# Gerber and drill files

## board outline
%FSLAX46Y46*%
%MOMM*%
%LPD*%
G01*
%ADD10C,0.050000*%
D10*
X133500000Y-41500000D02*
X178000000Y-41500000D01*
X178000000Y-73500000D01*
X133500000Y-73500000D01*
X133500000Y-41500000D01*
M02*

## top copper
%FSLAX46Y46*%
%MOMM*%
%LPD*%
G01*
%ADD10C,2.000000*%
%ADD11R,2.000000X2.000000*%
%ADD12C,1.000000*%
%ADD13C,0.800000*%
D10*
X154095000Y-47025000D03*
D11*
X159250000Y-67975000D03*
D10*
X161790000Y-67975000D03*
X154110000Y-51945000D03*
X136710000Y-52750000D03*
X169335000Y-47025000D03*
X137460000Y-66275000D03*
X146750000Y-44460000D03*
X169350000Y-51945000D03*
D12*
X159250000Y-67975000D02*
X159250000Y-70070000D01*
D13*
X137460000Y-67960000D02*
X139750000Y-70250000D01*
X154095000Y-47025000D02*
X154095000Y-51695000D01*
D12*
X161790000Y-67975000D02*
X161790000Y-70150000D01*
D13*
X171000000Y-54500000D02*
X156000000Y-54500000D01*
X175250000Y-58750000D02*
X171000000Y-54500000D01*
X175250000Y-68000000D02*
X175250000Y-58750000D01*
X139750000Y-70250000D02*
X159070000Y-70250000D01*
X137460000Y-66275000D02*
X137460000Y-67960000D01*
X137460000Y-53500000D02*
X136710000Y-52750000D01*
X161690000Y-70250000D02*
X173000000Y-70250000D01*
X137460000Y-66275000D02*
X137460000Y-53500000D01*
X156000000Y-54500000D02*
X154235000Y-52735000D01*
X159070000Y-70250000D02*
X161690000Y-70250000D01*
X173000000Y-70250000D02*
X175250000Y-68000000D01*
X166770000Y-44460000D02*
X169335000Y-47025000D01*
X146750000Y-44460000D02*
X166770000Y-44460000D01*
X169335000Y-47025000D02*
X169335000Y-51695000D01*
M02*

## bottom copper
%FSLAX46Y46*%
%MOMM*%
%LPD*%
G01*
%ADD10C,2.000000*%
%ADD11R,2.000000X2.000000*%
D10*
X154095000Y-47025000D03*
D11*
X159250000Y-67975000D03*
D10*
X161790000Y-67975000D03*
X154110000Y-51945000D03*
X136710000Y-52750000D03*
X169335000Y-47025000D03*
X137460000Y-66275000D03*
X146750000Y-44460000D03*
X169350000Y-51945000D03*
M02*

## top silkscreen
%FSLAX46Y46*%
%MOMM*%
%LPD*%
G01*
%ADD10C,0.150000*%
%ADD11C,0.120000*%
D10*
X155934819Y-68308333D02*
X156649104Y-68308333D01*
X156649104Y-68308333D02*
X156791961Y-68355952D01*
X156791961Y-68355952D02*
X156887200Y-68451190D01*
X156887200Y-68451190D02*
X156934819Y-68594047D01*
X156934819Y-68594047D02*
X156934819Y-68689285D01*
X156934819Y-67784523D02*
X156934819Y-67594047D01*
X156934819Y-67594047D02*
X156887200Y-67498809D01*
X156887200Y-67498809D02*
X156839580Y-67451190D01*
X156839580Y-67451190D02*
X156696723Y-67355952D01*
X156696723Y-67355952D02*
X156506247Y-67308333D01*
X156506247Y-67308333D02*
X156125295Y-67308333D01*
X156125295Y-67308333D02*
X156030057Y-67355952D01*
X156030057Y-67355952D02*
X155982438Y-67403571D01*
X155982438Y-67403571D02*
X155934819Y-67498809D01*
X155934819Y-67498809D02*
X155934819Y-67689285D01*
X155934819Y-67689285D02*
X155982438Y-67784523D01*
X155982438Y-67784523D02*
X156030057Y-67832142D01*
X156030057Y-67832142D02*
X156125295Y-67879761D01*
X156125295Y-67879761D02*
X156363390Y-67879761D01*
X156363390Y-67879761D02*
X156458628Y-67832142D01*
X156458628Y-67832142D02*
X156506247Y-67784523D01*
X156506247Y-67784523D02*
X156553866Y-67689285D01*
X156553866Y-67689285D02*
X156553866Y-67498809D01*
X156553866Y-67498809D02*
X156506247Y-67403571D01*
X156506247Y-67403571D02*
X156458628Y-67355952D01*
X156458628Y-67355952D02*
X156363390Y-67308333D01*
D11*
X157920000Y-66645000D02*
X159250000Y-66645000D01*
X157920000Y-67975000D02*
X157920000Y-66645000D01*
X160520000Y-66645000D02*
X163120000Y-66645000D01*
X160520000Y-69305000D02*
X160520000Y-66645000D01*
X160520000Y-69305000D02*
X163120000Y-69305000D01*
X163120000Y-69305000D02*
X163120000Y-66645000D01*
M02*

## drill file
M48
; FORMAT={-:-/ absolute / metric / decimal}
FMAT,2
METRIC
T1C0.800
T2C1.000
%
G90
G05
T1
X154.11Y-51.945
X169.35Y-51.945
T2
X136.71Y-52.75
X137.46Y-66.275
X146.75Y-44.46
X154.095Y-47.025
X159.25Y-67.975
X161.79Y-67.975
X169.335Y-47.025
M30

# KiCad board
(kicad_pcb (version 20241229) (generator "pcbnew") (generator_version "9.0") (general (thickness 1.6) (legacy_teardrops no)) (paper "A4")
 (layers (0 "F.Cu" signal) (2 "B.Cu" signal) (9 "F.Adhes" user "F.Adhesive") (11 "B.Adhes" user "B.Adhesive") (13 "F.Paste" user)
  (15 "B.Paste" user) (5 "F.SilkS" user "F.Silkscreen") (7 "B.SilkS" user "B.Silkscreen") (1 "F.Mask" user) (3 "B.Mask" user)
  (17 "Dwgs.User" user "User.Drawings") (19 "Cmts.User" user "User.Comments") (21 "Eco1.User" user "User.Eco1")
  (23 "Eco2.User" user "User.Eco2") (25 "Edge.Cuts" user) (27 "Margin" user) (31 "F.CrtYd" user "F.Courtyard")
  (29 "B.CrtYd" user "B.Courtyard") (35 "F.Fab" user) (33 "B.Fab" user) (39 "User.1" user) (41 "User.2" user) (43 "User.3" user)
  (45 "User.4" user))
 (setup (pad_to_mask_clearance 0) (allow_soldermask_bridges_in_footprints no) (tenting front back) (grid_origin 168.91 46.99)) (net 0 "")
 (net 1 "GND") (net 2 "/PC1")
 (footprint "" (layer "F.Cu") (at 149.16 46.74)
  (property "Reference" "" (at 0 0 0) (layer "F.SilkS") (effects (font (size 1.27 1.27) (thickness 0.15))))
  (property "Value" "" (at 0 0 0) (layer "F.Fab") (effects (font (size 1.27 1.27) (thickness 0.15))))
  (pad "8" thru_hole circle (at 4.935 0.285 270) (size 2 2) (drill 1) (layers "*.Cu" "*.Mask") (remove_unused_layers no) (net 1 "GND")))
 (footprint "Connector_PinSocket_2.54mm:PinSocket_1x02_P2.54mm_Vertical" (layer "F.Cu") (at 159.25 67.975 90)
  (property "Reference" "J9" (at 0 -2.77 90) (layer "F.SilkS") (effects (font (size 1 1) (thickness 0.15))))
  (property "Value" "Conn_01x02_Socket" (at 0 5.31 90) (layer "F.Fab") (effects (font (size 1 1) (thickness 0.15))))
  (fp_line (start 1.33 -1.33) (end 1.33 0) (stroke (width 0.12) (type solid)) (layer "F.SilkS"))
  (fp_line (start 0 -1.33) (end 1.33 -1.33) (stroke (width 0.12) (type solid)) (layer "F.SilkS"))
  (fp_line (start 1.33 1.27) (end 1.33 3.87) (stroke (width 0.12) (type solid)) (layer "F.SilkS"))
  (fp_line (start -1.33 1.27) (end 1.33 1.27) (stroke (width 0.12) (type solid)) (layer "F.SilkS"))
  (fp_line (start -1.33 1.27) (end -1.33 3.87) (stroke (width 0.12) (type solid)) (layer "F.SilkS"))
  (fp_line (start -1.33 3.87) (end 1.33 3.87) (stroke (width 0.12) (type solid)) (layer "F.SilkS"))
  (pad "1" thru_hole rect (at 0 0 90) (size 2 2) (drill 1) (layers "*.Cu" "*.Mask") (remove_unused_layers no) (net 1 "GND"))
  (pad "2" thru_hole circle (at 0 2.54 90) (size 2 2) (drill 1) (layers "*.Cu" "*.Mask") (remove_unused_layers no) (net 1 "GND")))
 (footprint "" (layer "F.Cu") (at 150.41 50.24)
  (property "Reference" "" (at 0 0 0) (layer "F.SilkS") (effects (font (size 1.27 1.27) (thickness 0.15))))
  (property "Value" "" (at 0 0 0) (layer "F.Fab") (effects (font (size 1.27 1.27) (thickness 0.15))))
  (pad "8" thru_hole circle (at 3.7 1.705 270) (size 2 2) (drill 0.8) (layers "*.Cu" "*.Mask") (remove_unused_layers no) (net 1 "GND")))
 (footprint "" (layer "F.Cu") (at 130.16 50.24)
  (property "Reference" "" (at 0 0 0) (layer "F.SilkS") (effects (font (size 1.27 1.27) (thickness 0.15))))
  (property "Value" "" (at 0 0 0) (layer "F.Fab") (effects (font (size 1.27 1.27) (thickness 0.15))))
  (pad "2" thru_hole circle (at 6.55 2.51 270) (size 2 2) (drill 1) (layers "*.Cu" "*.Mask") (remove_unused_layers no) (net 1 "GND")))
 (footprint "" (layer "F.Cu") (at 169.335 43.24)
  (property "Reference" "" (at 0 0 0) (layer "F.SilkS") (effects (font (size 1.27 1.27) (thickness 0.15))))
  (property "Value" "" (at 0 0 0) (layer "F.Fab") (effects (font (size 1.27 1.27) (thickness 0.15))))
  (pad "2" thru_hole circle (at 0 3.785 270) (size 2 2) (drill 1) (layers "*.Cu" "*.Mask") (remove_unused_layers no) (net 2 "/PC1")))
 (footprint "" (layer "F.Cu") (at 134.91 61.99)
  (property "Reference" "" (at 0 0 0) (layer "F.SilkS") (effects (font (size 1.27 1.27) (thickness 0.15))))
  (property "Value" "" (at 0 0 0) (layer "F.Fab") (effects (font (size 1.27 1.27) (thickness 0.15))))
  (pad "2" thru_hole circle (at 2.55 4.285 270) (size 2 2) (drill 1) (layers "*.Cu" "*.Mask") (remove_unused_layers no) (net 1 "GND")))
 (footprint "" (layer "F.Cu") (at 142.66 44.46)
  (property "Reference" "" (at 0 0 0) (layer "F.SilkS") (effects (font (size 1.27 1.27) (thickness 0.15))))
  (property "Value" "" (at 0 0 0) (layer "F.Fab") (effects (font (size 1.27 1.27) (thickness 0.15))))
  (pad "2" thru_hole circle (at 4.09 0 180) (size 2 2) (drill 1) (layers "*.Cu" "*.Mask") (remove_unused_layers no) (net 2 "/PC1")))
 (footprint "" (layer "F.Cu") (at 175.41 49.24)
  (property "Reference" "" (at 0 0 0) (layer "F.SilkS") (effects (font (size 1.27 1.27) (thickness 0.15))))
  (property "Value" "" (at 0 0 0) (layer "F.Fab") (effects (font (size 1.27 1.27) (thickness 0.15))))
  (pad "2" thru_hole circle (at -6.06 2.705 270) (size 2 2) (drill 0.8) (layers "*.Cu" "*.Mask") (remove_unused_layers no) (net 2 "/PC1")))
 (gr_rect (start 133.5 41.5) (end 178 73.5) (stroke (width 0.05) (type default)) (fill no) (locked yes) (layer "Edge.Cuts"))
 (segment (start 159.25 67.975) (end 159.25 70.07) (width 1) (locked yes) (layer "F.Cu") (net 1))
 (segment (start 137.46 67.96) (end 139.75 70.25) (width 0.8) (locked yes) (layer "F.Cu") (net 1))
 (segment (start 154.095 47.025) (end 154.095 51.695) (width 0.8) (locked yes) (layer "F.Cu") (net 1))
 (segment (start 161.79 67.975) (end 161.79 70.15) (width 1) (locked yes) (layer "F.Cu") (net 1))
 (segment (start 171 54.5) (end 156 54.5) (width 0.8) (locked yes) (layer "F.Cu") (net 1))
 (segment (start 175.25 58.75) (end 171 54.5) (width 0.8) (locked yes) (layer "F.Cu") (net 1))
 (segment (start 175.25 68) (end 175.25 58.75) (width 0.8) (locked yes) (layer "F.Cu") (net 1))
 (segment (start 139.75 70.25) (end 159.07 70.25) (width 0.8) (locked yes) (layer "F.Cu") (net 1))
 (segment (start 137.46 66.275) (end 137.46 67.96) (width 0.8) (locked yes) (layer "F.Cu") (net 1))
 (segment (start 137.46 53.5) (end 136.71 52.75) (width 0.8) (layer "F.Cu") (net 1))
 (segment (start 161.69 70.25) (end 173 70.25) (width 0.8) (locked yes) (layer "F.Cu") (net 1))
 (segment (start 137.46 66.275) (end 137.46 53.5) (width 0.8) (locked yes) (layer "F.Cu") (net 1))
 (segment (start 156 54.5) (end 154.235 52.735) (width 0.8) (locked yes) (layer "F.Cu") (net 1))
 (segment (start 159.07 70.25) (end 161.69 70.25) (width 0.8) (locked yes) (layer "F.Cu") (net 1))
 (segment (start 173 70.25) (end 175.25 68) (width 0.8) (locked yes) (layer "F.Cu") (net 1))
 (segment (start 166.77 44.46) (end 169.335 47.025) (width 0.8) (locked yes) (layer "F.Cu") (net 2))
 (segment (start 146.75 44.46) (end 166.77 44.46) (width 0.8) (locked yes) (layer "F.Cu") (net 2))
 (segment (start 169.335 47.025) (end 169.335 51.695) (width 0.8) (locked yes) (layer "F.Cu") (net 2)))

